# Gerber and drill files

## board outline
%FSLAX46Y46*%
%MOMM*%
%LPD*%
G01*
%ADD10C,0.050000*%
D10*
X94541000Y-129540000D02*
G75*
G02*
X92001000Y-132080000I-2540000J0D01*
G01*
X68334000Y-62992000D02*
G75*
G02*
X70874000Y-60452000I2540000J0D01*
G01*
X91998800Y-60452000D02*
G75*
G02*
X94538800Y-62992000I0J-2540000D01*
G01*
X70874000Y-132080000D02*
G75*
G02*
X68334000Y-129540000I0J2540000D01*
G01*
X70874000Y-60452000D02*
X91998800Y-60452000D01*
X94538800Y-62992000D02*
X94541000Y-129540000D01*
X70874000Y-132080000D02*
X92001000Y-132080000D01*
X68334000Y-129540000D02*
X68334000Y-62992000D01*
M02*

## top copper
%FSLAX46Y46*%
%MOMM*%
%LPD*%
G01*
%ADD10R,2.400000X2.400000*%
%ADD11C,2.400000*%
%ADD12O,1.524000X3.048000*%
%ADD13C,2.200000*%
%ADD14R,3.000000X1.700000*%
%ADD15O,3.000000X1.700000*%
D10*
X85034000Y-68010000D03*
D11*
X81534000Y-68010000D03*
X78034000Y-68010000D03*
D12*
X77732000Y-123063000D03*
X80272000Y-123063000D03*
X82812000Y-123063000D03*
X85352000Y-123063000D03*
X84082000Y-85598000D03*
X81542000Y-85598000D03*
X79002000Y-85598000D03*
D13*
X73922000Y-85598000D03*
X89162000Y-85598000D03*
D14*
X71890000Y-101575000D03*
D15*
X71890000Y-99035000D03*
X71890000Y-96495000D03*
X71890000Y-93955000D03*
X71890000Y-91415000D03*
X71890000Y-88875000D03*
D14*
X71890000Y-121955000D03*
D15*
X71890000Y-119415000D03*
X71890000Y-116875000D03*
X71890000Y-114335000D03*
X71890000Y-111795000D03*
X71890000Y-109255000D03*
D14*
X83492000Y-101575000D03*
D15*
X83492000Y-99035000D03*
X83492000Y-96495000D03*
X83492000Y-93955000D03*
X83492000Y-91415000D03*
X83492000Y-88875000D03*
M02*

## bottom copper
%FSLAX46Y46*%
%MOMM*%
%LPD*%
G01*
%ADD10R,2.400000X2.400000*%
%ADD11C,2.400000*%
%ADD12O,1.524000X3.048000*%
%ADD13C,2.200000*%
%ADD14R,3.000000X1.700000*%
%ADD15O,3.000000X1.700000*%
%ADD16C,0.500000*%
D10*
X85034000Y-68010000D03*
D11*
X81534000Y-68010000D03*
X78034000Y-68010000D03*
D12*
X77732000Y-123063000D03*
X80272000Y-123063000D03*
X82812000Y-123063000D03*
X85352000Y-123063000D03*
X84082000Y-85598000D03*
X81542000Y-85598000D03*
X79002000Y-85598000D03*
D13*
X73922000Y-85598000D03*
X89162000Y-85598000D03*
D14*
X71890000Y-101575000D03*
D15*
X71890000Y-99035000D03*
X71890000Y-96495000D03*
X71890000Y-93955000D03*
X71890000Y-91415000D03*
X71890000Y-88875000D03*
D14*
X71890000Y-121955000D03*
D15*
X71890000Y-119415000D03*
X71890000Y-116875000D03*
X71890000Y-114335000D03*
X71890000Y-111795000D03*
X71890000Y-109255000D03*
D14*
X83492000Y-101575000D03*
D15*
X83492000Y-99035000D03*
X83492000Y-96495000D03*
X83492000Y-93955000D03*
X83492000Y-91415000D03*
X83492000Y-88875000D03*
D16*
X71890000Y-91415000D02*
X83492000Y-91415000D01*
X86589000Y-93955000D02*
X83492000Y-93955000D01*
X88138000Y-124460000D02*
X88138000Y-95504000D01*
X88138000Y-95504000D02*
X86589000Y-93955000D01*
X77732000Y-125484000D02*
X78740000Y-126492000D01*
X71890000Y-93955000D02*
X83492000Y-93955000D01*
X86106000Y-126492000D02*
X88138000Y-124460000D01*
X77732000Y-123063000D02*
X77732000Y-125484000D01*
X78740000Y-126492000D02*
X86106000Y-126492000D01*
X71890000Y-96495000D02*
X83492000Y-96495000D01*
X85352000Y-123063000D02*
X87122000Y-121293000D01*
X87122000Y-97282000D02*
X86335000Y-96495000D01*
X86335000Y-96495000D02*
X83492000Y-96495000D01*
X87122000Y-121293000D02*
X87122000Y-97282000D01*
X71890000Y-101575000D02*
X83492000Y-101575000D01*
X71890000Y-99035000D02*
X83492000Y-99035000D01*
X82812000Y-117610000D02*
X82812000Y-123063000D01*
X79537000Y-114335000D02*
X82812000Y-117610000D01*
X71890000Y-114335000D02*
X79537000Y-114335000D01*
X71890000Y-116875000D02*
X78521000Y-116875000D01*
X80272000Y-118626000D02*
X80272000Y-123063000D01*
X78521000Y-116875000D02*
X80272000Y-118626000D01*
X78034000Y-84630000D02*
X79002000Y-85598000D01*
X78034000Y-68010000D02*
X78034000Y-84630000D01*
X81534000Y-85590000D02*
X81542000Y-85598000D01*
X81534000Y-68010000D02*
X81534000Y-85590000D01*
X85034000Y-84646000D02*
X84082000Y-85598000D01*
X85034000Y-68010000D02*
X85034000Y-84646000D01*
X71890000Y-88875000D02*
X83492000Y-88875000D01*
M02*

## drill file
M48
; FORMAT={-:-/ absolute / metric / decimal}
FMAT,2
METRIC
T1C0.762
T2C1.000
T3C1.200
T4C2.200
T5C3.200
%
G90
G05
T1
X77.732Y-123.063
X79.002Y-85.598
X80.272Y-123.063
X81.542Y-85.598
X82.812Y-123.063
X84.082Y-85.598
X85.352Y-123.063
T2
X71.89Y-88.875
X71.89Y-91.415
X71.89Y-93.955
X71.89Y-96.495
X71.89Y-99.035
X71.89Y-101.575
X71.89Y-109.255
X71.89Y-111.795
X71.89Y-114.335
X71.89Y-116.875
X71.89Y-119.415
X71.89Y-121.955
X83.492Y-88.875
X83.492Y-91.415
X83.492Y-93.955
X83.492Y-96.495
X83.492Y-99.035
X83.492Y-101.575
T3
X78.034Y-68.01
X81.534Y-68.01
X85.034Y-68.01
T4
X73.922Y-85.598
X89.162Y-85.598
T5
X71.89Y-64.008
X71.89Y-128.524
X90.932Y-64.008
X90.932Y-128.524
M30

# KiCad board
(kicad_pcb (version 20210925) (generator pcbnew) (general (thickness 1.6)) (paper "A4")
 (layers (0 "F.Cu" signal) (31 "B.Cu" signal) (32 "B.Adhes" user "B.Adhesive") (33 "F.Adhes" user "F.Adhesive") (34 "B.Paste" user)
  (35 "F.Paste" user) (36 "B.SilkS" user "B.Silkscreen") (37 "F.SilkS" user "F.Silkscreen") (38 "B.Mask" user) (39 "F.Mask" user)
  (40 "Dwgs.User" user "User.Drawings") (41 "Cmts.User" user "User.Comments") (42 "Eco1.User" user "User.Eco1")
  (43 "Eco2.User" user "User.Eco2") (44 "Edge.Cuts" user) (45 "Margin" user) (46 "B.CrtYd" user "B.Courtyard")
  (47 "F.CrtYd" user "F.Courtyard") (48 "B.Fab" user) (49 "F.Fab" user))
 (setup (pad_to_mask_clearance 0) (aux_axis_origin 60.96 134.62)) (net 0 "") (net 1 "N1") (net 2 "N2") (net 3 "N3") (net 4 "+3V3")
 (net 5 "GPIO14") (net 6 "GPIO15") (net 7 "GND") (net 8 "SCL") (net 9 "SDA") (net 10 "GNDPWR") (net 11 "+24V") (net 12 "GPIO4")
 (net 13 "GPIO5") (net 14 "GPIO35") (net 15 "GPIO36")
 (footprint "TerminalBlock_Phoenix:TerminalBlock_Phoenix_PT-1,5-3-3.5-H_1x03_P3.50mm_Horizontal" (layer "F.Cu") (at 85.034 68.01 180)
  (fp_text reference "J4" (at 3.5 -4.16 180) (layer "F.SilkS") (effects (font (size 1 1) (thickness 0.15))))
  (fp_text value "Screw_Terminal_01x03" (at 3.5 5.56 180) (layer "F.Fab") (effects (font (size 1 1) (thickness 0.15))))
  (pad "1" thru_hole rect locked (at 0 0 180) (size 2.4 2.4) (drill 1.2) (layers *.Cu *.Mask) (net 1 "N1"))
  (pad "2" thru_hole circle locked (at 3.5 0 180) (size 2.4 2.4) (drill 1.2) (layers *.Cu *.Mask) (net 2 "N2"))
  (pad "3" thru_hole circle locked (at 7 0 180) (size 2.4 2.4) (drill 1.2) (layers *.Cu *.Mask) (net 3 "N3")))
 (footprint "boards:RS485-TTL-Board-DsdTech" (layer "F.Cu") (at 81.542 102.108)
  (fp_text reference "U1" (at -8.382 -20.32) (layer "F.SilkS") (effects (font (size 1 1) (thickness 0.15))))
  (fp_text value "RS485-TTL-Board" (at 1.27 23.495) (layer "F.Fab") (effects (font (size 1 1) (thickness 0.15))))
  (pad "" smd circle locked (at -7.62 22.225) (size 1 1) (layers "F.Mask") (die_length 4))
  (pad "" smd circle locked (at 7.62 22.225) (size 1 1) (layers "F.Mask") (die_length 4))
  (pad "1" thru_hole oval locked (at -3.81 20.955) (size 1.524 3.048) (drill 0.762) (layers *.Cu *.Mask) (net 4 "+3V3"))
  (pad "2" thru_hole oval locked (at -1.27 20.955) (size 1.524 3.048) (drill 0.762) (layers *.Cu *.Mask) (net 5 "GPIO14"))
  (pad "3" thru_hole oval locked (at 1.27 20.955) (size 1.524 3.048) (drill 0.762) (layers *.Cu *.Mask) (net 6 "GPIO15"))
  (pad "4" thru_hole oval locked (at 3.81 20.955) (size 1.524 3.048) (drill 0.762) (layers *.Cu *.Mask) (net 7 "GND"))
  (pad "5" thru_hole oval locked (at 2.54 -16.51) (size 1.524 3.048) (drill 0.762) (layers *.Cu *.Mask) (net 1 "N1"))
  (pad "6" thru_hole oval locked (at 0 -16.51) (size 1.524 3.048) (drill 0.762) (layers *.Cu *.Mask) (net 2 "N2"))
  (pad "7" thru_hole oval locked (at -2.54 -16.51) (size 1.524 3.048) (drill 0.762) (layers *.Cu *.Mask) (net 3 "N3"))
  (pad "8" thru_hole circle locked (at -7.62 -16.51) (size 2.2 2.2) (drill 2.2) (layers *.Cu *.Mask) (die_length 4))
  (pad "8" thru_hole circle locked (at 7.62 -16.51) (size 2.2 2.2) (drill 2.2) (layers *.Cu *.Mask) (die_length 4)))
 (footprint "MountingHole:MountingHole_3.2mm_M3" (layer "F.Cu") (at 90.932 64.008)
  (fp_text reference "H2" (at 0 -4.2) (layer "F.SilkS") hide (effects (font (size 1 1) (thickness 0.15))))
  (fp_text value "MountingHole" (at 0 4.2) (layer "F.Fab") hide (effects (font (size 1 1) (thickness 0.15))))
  (pad "" np_thru_hole circle locked (at 0 0) (size 3.2 3.2) (drill 3.2) (layers *.Cu *.Mask)))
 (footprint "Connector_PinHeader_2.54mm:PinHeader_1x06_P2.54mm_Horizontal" (layer "F.Cu") (at 71.89 101.575 180)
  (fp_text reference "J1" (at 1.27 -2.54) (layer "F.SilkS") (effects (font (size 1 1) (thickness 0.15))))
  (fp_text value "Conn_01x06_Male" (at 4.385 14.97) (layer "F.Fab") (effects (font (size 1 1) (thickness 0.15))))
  (pad "1" thru_hole rect locked (at 0 0 180) (size 3 1.7) (drill 1) (layers *.Cu *.Mask) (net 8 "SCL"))
  (pad "2" thru_hole oval locked (at 0 2.54 180) (size 3 1.7) (drill 1) (layers *.Cu *.Mask) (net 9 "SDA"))
  (pad "3" thru_hole oval locked (at 0 5.08 180) (size 3 1.7) (drill 1) (layers *.Cu *.Mask) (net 7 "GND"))
  (pad "4" thru_hole oval locked (at 0 7.62 180) (size 3 1.7) (drill 1) (layers *.Cu *.Mask) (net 4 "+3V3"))
  (pad "5" thru_hole oval locked (at 0 10.16 180) (size 3 1.7) (drill 1) (layers *.Cu *.Mask) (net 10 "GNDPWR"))
  (pad "6" thru_hole oval locked (at 0 12.7 180) (size 3 1.7) (drill 1) (layers *.Cu *.Mask) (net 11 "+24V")))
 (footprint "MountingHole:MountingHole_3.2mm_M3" (layer "F.Cu") (at 90.932 128.524)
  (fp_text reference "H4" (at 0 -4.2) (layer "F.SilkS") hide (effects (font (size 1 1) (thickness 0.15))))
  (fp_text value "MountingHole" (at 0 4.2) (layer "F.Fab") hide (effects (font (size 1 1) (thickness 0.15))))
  (pad "" np_thru_hole circle locked (at 0 0) (size 3.2 3.2) (drill 3.2) (layers *.Cu *.Mask)))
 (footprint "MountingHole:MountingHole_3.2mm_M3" (layer "F.Cu") (at 71.89 128.524)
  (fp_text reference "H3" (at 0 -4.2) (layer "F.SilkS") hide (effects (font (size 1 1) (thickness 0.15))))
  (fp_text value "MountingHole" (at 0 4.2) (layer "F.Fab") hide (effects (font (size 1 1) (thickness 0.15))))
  (pad "" np_thru_hole circle locked (at 0 0) (size 3.2 3.2) (drill 3.2) (layers *.Cu *.Mask)))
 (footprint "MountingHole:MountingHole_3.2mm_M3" (layer "F.Cu") (at 71.89 64.008)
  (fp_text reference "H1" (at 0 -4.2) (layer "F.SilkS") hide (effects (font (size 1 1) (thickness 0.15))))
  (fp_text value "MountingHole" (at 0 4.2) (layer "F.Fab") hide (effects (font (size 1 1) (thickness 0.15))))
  (pad "" np_thru_hole circle locked (at 0 0) (size 3.2 3.2) (drill 3.2) (layers *.Cu *.Mask)))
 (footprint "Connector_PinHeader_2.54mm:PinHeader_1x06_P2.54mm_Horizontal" (layer "F.Cu") (at 71.89 121.955 180)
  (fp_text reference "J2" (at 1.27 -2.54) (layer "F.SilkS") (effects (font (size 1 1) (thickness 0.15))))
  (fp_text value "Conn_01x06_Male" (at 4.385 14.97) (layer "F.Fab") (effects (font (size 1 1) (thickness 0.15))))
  (pad "1" thru_hole rect locked (at 0 0 180) (size 3 1.7) (drill 1) (layers *.Cu *.Mask) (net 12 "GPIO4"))
  (pad "2" thru_hole oval locked (at 0 2.54 180) (size 3 1.7) (drill 1) (layers *.Cu *.Mask) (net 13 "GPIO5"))
  (pad "3" thru_hole oval locked (at 0 5.08 180) (size 3 1.7) (drill 1) (layers *.Cu *.Mask) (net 5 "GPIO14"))
  (pad "4" thru_hole oval locked (at 0 7.62 180) (size 3 1.7) (drill 1) (layers *.Cu *.Mask) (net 6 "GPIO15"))
  (pad "5" thru_hole oval locked (at 0 10.16 180) (size 3 1.7) (drill 1) (layers *.Cu *.Mask) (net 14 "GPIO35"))
  (pad "6" thru_hole oval locked (at 0 12.7 180) (size 3 1.7) (drill 1) (layers *.Cu *.Mask) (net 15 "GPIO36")))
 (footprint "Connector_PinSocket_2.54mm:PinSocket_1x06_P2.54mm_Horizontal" (layer "F.Cu") (at 83.492 101.575 180)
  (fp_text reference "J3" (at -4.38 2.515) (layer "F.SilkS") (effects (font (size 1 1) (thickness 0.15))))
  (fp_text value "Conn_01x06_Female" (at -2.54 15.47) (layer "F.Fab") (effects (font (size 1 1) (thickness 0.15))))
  (pad "1" thru_hole rect locked (at 0 0 180) (size 3 1.7) (drill 1) (layers *.Cu *.Mask) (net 8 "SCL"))
  (pad "2" thru_hole oval locked (at 0 2.54 180) (size 3 1.7) (drill 1) (layers *.Cu *.Mask) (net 9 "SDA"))
  (pad "3" thru_hole oval locked (at 0 5.08 180) (size 3 1.7) (drill 1) (layers *.Cu *.Mask) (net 7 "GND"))
  (pad "4" thru_hole oval locked (at 0 7.62 180) (size 3 1.7) (drill 1) (layers *.Cu *.Mask) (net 4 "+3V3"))
  (pad "5" thru_hole oval locked (at 0 10.16 180) (size 3 1.7) (drill 1) (layers *.Cu *.Mask) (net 10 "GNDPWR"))
  (pad "6" thru_hole oval locked (at 0 12.7 180) (size 3 1.7) (drill 1) (layers *.Cu *.Mask) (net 11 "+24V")))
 (gr_arc (start 92.001 129.54) (end 92.001 132.08) (angle -90) (layer "Edge.Cuts") (width 0.05))
 (gr_arc (start 70.874 62.992) (end 70.874 60.452) (angle -90) (layer "Edge.Cuts") (width 0.05))
 (gr_arc (start 91.9988 62.992) (end 94.5388 62.992) (angle -90) (layer "Edge.Cuts") (width 0.05))
 (gr_arc (start 70.874 129.54) (end 68.334 129.54) (angle -90) (layer "Edge.Cuts") (width 0.05))
 (gr_line (start 70.874 60.452) (end 91.9988 60.452) (layer "Edge.Cuts") (width 0.05))
 (gr_line (start 94.5388 62.992) (end 94.541 129.54) (layer "Edge.Cuts") (width 0.05))
 (gr_line (start 70.874 132.08) (end 92.001 132.08) (layer "Edge.Cuts") (width 0.05))
 (gr_line (start 68.334 129.54) (end 68.334 62.992) (layer "Edge.Cuts") (width 0.05))
 (segment (start 71.89 91.415) (end 83.492 91.415) (width 0.5) (layer "B.Cu") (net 10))
 (segment (start 86.589 93.955) (end 83.492 93.955) (width 0.5) (layer "B.Cu") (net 4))
 (segment (start 88.138 124.46) (end 88.138 95.504) (width 0.5) (layer "B.Cu") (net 4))
 (segment (start 88.138 95.504) (end 86.589 93.955) (width 0.5) (layer "B.Cu") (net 4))
 (segment (start 77.732 125.484) (end 78.74 126.492) (width 0.5) (layer "B.Cu") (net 4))
 (segment (start 71.89 93.955) (end 83.492 93.955) (width 0.5) (layer "B.Cu") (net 4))
 (segment (start 86.106 126.492) (end 88.138 124.46) (width 0.5) (layer "B.Cu") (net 4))
 (segment (start 77.732 123.063) (end 77.732 125.484) (width 0.5) (layer "B.Cu") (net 4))
 (segment (start 78.74 126.492) (end 86.106 126.492) (width 0.5) (layer "B.Cu") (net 4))
 (segment (start 71.89 96.495) (end 83.492 96.495) (width 0.5) (layer "B.Cu") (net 7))
 (segment (start 85.352 123.063) (end 87.122 121.293) (width 0.5) (layer "B.Cu") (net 7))
 (segment (start 87.122 97.282) (end 86.335 96.495) (width 0.5) (layer "B.Cu") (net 7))
 (segment (start 86.335 96.495) (end 83.492 96.495) (width 0.5) (layer "B.Cu") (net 7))
 (segment (start 87.122 121.293) (end 87.122 97.282) (width 0.5) (layer "B.Cu") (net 7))
 (segment (start 71.89 101.575) (end 83.492 101.575) (width 0.5) (layer "B.Cu") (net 8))
 (segment (start 71.89 99.035) (end 83.492 99.035) (width 0.5) (layer "B.Cu") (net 9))
 (segment (start 82.812 117.61) (end 82.812 123.063) (width 0.5) (layer "B.Cu") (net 6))
 (segment (start 79.537 114.335) (end 82.812 117.61) (width 0.5) (layer "B.Cu") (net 6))
 (segment (start 71.89 114.335) (end 79.537 114.335) (width 0.5) (layer "B.Cu") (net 6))
 (segment (start 71.89 116.875) (end 78.521 116.875) (width 0.5) (layer "B.Cu") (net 5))
 (segment (start 80.272 118.626) (end 80.272 123.063) (width 0.5) (layer "B.Cu") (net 5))
 (segment (start 78.521 116.875) (end 80.272 118.626) (width 0.5) (layer "B.Cu") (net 5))
 (segment (start 78.034 84.63) (end 79.002 85.598) (width 0.5) (layer "B.Cu") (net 3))
 (segment (start 78.034 68.01) (end 78.034 84.63) (width 0.5) (layer "B.Cu") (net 3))
 (segment (start 81.534 85.59) (end 81.542 85.598) (width 0.5) (layer "B.Cu") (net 2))
 (segment (start 81.534 68.01) (end 81.534 85.59) (width 0.5) (layer "B.Cu") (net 2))
 (segment (start 85.034 84.646) (end 84.082 85.598) (width 0.5) (layer "B.Cu") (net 1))
 (segment (start 85.034 68.01) (end 85.034 84.646) (width 0.5) (layer "B.Cu") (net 1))
 (segment (start 71.89 88.875) (end 83.492 88.875) (width 0.5) (layer "B.Cu") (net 11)))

